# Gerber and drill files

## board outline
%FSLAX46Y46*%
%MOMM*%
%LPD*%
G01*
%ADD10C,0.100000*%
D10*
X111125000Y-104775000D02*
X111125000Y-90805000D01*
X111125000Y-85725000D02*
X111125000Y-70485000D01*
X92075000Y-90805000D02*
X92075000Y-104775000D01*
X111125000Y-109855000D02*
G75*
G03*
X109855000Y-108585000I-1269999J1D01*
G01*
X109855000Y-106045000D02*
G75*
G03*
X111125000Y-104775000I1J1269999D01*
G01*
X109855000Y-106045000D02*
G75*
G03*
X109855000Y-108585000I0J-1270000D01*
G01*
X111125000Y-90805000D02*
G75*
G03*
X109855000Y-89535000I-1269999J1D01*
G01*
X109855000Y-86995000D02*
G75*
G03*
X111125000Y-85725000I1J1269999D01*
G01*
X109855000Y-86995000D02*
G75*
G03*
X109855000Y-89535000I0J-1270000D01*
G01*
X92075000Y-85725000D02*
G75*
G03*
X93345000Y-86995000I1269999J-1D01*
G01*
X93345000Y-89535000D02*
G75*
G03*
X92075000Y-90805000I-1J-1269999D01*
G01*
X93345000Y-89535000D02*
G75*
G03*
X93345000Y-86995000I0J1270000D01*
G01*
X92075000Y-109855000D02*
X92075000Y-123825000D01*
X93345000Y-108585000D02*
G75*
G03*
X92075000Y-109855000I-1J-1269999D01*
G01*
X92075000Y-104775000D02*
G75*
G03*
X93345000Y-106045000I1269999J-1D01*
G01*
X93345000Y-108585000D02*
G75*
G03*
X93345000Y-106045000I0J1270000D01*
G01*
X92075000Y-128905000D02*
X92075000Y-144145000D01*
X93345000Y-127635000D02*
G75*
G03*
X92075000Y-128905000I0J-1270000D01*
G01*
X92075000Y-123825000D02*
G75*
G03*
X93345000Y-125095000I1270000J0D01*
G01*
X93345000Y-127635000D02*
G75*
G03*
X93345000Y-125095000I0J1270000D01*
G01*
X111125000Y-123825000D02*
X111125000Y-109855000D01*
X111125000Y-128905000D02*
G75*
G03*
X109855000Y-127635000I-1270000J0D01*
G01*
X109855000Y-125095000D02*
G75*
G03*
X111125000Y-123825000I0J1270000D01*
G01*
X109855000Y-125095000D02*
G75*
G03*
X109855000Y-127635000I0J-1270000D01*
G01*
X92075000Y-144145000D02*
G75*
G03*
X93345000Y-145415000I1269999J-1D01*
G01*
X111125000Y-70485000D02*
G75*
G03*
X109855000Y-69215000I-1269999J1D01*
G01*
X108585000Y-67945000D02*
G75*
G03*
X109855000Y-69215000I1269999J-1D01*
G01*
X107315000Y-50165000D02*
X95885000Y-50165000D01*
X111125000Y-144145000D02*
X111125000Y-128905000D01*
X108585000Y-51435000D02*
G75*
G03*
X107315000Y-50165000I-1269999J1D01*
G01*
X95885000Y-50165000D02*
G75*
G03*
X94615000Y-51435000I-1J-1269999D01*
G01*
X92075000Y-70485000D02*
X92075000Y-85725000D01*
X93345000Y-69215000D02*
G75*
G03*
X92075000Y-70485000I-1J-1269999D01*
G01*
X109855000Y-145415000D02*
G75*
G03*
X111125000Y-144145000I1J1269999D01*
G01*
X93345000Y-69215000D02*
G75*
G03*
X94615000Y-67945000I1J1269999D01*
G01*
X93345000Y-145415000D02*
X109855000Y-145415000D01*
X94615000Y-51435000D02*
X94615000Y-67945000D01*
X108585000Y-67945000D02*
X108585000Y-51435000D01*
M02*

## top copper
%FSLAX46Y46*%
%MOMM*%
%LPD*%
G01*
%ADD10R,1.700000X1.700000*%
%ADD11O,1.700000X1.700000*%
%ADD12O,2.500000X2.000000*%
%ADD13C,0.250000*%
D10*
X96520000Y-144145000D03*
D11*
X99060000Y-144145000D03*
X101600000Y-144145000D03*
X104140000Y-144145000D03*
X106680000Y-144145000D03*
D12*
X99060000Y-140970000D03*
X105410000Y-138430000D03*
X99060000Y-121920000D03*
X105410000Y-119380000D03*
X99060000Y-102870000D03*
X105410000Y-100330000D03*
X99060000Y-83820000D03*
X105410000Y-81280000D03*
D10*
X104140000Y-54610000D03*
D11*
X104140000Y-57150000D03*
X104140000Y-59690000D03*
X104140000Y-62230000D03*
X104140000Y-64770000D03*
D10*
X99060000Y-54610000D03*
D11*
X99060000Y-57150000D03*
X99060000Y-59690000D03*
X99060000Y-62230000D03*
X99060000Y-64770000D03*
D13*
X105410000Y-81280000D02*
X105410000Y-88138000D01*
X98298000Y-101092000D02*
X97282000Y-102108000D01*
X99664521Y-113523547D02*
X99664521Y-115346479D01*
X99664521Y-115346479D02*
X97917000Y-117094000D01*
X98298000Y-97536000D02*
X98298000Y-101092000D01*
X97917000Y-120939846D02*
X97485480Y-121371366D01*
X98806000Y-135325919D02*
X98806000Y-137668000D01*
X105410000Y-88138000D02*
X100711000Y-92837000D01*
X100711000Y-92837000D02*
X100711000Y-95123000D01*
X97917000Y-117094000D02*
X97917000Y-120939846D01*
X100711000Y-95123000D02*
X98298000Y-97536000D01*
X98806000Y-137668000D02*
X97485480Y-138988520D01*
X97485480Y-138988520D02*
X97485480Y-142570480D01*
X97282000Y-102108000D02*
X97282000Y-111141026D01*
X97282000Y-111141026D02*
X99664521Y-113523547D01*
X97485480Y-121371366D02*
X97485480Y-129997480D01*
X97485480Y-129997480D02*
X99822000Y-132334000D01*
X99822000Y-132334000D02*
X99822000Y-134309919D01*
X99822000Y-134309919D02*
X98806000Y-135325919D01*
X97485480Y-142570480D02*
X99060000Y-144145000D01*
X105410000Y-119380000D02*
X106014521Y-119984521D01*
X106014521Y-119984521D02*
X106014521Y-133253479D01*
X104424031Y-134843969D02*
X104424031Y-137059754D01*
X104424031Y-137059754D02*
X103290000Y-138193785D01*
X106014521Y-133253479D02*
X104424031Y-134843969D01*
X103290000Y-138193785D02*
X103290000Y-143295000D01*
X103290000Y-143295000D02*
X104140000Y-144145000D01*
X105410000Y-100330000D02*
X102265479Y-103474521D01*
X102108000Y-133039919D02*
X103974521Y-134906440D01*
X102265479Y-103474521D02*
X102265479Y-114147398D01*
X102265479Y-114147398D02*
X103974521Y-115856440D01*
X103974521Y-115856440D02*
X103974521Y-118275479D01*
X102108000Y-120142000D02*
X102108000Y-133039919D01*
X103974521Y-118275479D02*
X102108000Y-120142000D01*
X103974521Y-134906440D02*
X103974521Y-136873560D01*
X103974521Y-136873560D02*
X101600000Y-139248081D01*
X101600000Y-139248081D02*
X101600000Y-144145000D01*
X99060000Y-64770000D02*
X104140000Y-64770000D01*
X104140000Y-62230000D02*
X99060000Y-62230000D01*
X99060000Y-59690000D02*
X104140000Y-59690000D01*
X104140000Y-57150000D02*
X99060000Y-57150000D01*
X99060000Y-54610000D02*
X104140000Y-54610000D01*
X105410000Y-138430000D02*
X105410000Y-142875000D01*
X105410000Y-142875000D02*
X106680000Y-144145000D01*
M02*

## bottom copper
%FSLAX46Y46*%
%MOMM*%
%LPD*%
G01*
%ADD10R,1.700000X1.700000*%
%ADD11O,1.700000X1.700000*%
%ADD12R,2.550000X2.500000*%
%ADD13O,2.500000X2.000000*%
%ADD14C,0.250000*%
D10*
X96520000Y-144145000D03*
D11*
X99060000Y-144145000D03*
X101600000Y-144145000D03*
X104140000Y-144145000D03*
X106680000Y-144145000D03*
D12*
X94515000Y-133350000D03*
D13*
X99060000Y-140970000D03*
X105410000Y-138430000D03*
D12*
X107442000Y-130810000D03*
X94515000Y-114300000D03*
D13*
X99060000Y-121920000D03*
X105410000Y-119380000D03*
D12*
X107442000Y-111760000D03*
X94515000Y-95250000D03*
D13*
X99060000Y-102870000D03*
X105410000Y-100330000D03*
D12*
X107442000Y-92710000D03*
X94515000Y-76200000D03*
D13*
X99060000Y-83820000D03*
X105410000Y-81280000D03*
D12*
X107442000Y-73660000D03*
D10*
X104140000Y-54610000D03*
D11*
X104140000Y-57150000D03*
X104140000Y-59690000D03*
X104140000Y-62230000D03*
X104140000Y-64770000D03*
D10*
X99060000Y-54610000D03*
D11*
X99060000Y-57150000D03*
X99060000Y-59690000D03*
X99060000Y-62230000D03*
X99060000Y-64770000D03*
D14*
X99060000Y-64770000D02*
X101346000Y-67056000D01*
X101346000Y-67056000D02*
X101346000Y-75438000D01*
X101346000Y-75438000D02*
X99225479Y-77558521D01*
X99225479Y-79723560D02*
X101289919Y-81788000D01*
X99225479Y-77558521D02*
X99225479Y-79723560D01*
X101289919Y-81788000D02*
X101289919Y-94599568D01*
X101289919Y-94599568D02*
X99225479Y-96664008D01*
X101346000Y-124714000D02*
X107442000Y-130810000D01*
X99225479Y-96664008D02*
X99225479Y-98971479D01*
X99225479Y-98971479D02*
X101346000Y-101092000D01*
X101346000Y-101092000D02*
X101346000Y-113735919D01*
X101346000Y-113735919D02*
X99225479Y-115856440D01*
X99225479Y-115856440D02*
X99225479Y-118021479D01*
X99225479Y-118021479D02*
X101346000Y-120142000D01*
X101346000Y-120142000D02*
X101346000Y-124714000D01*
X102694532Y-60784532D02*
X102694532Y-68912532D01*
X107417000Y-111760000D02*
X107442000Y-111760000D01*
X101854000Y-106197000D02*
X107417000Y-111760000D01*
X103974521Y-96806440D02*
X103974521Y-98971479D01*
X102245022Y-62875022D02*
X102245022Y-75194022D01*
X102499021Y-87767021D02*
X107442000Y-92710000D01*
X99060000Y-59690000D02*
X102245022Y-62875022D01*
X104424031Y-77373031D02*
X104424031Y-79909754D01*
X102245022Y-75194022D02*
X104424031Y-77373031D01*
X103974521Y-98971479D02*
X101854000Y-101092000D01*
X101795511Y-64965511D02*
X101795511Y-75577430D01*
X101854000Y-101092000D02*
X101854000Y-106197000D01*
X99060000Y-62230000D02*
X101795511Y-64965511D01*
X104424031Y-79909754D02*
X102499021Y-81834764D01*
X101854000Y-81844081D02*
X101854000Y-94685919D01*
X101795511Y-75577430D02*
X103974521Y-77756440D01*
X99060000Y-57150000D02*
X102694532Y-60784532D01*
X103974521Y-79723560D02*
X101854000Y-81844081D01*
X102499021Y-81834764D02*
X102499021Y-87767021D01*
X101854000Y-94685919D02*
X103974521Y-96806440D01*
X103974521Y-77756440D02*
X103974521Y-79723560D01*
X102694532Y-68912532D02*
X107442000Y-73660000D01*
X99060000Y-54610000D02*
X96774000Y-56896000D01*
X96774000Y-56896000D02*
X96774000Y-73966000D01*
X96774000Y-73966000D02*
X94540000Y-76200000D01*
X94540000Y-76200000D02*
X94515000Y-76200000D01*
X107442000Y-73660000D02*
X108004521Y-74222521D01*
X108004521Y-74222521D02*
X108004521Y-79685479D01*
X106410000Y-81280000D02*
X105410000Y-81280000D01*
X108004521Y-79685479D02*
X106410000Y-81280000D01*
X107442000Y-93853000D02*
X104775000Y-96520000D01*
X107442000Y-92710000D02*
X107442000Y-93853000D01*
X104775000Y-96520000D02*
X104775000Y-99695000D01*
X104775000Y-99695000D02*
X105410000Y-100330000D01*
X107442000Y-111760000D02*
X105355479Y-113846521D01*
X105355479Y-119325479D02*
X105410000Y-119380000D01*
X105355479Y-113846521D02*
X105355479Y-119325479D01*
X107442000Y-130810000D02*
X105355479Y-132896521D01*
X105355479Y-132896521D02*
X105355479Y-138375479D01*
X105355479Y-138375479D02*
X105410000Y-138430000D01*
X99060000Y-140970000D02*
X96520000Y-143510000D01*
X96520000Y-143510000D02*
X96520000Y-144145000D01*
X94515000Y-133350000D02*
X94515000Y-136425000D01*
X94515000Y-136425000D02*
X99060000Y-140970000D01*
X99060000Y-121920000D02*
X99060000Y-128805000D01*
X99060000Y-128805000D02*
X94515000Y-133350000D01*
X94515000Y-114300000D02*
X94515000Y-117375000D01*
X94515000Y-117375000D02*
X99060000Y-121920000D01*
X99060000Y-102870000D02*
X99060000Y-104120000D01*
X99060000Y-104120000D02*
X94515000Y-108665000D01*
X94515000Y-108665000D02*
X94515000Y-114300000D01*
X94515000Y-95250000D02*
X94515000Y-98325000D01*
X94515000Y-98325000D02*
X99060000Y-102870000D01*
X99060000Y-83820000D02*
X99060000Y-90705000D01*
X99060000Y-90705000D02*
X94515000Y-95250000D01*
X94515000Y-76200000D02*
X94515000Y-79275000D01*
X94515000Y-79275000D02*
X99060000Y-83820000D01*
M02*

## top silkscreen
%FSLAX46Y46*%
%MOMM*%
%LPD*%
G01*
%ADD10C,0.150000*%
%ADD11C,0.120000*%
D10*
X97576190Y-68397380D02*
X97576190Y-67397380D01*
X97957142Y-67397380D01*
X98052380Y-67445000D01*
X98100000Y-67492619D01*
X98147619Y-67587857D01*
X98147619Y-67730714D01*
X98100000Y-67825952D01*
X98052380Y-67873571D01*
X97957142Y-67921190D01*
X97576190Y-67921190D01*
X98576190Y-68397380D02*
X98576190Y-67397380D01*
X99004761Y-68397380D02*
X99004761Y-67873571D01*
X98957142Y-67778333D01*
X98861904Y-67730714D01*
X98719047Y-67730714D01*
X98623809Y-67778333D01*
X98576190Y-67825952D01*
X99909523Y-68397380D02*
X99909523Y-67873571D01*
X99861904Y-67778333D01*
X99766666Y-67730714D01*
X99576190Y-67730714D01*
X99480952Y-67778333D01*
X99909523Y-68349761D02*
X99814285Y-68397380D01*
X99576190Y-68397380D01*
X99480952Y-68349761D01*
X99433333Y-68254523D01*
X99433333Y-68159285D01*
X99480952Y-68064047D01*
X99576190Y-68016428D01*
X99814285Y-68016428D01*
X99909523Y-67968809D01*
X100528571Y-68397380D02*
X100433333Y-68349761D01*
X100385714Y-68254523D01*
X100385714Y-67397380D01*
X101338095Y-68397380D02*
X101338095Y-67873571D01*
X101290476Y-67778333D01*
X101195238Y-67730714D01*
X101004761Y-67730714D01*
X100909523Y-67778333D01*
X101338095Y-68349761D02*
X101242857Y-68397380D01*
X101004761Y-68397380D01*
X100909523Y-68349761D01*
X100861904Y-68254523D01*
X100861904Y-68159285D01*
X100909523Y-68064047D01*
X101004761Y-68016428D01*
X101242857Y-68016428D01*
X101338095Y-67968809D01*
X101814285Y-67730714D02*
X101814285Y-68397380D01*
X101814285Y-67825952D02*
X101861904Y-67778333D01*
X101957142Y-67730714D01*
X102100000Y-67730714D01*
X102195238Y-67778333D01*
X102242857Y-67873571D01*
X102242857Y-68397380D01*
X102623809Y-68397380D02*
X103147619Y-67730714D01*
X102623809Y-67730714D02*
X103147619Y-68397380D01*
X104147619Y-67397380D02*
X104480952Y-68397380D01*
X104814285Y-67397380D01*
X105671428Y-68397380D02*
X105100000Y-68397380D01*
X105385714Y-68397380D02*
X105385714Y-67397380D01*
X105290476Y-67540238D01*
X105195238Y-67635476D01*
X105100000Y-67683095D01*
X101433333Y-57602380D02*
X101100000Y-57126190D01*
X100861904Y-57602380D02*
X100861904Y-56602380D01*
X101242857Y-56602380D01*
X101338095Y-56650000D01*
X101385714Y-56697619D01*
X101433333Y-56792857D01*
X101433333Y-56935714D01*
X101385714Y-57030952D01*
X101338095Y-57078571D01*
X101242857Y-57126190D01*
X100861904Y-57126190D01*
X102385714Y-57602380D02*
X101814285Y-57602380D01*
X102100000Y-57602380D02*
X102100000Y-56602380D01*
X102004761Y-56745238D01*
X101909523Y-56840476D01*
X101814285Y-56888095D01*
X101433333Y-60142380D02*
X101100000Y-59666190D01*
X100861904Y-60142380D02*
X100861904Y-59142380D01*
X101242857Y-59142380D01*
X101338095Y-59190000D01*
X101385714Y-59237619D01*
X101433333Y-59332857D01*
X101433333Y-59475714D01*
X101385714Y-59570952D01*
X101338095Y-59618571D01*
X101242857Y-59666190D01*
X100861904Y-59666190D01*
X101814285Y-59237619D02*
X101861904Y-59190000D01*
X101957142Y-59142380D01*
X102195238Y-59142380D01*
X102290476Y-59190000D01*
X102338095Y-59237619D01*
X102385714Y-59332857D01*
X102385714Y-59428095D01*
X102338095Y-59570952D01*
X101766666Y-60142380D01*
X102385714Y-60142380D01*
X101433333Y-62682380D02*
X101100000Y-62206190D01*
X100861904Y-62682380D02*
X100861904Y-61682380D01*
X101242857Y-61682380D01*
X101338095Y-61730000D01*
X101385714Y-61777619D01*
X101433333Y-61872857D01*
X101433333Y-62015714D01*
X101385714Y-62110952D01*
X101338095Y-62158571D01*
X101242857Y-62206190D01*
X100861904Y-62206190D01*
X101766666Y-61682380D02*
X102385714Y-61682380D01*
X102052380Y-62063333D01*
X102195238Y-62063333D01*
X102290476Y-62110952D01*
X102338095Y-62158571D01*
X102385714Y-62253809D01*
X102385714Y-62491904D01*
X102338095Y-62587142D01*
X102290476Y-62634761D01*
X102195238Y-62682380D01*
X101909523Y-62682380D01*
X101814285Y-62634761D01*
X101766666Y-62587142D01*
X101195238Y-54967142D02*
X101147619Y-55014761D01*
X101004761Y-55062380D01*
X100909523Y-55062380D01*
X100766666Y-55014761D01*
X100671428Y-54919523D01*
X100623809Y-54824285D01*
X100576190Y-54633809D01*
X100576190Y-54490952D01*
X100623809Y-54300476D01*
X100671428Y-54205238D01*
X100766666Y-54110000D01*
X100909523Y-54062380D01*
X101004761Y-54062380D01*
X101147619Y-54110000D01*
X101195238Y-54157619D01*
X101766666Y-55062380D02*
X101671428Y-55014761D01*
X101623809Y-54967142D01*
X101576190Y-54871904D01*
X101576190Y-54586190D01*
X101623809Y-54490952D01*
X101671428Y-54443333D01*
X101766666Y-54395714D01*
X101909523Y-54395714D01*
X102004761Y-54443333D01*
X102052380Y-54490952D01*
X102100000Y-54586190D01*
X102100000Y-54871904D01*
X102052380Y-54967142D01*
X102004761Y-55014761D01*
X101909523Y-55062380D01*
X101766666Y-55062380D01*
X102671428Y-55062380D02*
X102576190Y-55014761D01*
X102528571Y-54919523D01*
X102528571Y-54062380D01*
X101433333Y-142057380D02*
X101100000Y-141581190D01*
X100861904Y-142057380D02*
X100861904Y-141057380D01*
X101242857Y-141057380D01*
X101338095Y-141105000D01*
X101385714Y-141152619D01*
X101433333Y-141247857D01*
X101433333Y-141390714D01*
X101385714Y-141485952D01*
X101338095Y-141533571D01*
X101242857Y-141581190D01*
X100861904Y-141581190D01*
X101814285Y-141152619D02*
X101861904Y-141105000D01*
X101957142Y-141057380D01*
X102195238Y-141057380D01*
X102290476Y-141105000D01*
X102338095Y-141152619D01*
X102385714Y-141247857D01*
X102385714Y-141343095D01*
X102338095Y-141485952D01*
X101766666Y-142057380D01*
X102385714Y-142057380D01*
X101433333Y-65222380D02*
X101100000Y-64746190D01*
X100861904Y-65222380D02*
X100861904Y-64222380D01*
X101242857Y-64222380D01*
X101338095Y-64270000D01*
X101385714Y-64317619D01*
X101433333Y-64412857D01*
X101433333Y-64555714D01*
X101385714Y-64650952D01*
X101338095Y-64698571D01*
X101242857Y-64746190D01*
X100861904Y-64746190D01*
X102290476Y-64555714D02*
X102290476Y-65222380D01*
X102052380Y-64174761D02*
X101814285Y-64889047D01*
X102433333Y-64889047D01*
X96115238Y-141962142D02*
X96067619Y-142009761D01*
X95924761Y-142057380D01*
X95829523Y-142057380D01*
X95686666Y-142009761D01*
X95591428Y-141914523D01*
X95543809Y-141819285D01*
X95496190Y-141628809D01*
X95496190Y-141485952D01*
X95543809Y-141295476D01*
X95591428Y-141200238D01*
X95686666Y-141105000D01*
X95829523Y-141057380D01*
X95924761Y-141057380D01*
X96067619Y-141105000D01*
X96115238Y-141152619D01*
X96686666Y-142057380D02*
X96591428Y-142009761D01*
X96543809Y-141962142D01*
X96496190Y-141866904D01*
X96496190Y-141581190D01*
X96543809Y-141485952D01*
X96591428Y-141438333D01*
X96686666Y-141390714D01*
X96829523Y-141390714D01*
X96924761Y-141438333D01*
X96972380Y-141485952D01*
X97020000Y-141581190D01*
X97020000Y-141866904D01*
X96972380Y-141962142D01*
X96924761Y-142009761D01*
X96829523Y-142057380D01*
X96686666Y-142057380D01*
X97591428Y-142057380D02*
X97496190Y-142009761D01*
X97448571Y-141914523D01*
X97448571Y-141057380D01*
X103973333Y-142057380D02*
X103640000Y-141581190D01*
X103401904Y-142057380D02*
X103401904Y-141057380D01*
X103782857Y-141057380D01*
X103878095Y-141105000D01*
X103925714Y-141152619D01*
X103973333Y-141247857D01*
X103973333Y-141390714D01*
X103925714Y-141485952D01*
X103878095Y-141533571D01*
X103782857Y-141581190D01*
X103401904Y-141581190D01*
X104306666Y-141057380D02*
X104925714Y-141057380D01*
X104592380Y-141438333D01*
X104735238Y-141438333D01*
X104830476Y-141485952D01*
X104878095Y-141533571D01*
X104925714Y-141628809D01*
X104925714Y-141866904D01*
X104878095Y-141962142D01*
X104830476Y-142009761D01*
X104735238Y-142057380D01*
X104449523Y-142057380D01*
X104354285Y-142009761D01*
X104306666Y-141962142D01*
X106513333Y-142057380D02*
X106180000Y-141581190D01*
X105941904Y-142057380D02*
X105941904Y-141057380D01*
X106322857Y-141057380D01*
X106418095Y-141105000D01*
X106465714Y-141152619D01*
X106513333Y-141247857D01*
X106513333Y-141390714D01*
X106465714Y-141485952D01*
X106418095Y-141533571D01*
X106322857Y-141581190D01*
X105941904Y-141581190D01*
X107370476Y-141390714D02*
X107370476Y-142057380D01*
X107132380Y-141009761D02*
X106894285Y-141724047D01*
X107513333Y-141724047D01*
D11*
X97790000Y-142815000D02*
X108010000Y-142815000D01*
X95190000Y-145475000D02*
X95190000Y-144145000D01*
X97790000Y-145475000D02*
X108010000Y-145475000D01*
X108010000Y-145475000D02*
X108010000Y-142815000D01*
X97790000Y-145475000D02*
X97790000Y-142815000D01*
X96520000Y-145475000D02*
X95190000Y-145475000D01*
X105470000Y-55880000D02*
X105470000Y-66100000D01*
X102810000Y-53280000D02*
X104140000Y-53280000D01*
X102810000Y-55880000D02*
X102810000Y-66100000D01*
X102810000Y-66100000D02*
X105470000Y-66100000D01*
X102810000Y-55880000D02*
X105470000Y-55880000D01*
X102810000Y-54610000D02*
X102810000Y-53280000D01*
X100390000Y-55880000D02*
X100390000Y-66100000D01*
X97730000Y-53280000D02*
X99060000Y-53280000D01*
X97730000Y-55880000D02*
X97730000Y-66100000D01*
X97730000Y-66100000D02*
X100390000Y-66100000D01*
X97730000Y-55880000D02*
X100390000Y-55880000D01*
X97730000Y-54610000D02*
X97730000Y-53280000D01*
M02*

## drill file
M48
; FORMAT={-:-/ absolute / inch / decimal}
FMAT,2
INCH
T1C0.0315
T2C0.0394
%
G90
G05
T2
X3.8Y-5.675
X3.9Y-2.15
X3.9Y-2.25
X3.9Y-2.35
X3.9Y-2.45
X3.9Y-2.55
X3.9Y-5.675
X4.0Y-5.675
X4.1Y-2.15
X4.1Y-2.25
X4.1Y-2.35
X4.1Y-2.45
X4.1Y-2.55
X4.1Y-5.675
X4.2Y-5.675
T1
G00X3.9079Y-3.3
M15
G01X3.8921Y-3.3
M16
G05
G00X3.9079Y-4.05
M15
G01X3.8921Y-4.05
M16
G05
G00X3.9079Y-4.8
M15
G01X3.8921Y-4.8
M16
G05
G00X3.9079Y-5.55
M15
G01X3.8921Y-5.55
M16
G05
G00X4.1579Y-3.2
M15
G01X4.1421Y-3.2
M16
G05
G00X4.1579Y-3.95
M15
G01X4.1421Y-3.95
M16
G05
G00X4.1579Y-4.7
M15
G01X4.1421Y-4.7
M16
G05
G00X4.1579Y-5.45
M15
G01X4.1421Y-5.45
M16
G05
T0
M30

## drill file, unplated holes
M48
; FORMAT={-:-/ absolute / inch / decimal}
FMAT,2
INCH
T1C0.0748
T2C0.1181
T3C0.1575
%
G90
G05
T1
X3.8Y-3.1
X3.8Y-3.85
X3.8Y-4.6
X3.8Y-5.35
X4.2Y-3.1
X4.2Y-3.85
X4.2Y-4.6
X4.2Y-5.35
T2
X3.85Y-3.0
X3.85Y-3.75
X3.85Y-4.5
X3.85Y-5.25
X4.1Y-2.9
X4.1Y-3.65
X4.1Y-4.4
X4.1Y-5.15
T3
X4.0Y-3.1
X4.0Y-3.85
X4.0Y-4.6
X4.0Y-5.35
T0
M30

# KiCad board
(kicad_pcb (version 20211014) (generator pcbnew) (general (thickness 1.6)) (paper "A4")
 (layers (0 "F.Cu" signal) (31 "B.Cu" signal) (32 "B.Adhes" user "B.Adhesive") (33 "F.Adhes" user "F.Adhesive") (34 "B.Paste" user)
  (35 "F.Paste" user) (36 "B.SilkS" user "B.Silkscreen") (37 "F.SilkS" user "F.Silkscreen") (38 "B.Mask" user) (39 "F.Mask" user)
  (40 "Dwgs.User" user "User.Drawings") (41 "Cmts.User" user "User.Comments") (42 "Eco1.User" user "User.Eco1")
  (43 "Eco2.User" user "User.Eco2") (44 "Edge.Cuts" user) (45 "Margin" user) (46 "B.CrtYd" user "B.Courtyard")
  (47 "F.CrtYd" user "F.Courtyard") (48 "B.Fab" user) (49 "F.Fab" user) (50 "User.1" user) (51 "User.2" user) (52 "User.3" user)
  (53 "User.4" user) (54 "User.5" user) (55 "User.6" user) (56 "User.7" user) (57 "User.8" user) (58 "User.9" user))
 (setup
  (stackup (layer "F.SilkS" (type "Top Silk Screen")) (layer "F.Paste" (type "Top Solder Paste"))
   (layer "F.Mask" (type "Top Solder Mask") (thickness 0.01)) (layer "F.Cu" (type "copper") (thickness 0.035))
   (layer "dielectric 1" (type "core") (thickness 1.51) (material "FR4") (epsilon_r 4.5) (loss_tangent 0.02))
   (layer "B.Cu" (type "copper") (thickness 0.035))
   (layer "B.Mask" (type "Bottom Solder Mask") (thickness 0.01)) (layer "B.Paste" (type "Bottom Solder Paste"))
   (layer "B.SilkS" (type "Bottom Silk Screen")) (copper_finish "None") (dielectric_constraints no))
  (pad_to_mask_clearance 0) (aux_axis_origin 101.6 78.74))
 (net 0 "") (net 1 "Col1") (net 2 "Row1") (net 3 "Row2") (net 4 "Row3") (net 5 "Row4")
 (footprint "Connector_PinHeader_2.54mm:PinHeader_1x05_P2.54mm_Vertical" (layer "F.Cu") (at 104.14 54.61)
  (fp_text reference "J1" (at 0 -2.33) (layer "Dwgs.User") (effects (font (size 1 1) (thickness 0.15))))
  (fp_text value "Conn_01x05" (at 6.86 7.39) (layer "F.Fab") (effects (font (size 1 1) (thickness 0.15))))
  (fp_line (start -1.33 -1.33) (end 0 -1.33) (layer "F.SilkS") (width 0.12))
  (fp_line (start -1.33 1.27) (end -1.33 11.49) (layer "F.SilkS") (width 0.12))
  (fp_line (start -1.33 11.49) (end 1.33 11.49) (layer "F.SilkS") (width 0.12))
  (fp_line (start -1.33 0) (end -1.33 -1.33) (layer "F.SilkS") (width 0.12))
  (fp_line (start -1.33 1.27) (end 1.33 1.27) (layer "F.SilkS") (width 0.12))
  (fp_line (start 1.33 1.27) (end 1.33 11.49) (layer "F.SilkS") (width 0.12))
  (pad "1" thru_hole rect (at 0 0) (size 1.7 1.7) (drill 1) (layers *.Cu *.Mask) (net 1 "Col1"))
  (pad "2" thru_hole oval (at 0 2.54) (size 1.7 1.7) (drill 1) (layers *.Cu *.Mask) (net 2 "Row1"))
  (pad "3" thru_hole oval (at 0 5.08) (size 1.7 1.7) (drill 1) (layers *.Cu *.Mask) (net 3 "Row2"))
  (pad "4" thru_hole oval (at 0 7.62) (size 1.7 1.7) (drill 1) (layers *.Cu *.Mask) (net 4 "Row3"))
  (pad "5" thru_hole oval (at 0 10.16) (size 1.7 1.7) (drill 1) (layers *.Cu *.Mask) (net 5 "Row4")))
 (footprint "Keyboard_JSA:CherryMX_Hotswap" (layer "F.Cu") (at 101.6 116.84)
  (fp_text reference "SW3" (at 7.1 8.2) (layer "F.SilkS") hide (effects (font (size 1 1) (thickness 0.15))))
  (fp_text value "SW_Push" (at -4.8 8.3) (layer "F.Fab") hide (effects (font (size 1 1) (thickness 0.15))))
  (pad "" np_thru_hole circle (at -5.08 0) (size 1.9 1.9) (drill 1.9) (layers *.Cu *.Mask))
  (pad "" np_thru_hole circle (at 2.54 -5.08) (size 3 3) (drill 3) (layers *.Cu *.Mask))
  (pad "" np_thru_hole circle (at 0 0) (size 4 4) (drill 4) (layers F&B.Cu *.Mask))
  (pad "" np_thru_hole circle (at 5.08 0) (size 1.9 1.9) (drill 1.9) (layers *.Cu *.Mask))
  (pad "" np_thru_hole circle (at -3.81 -2.54) (size 3 3) (drill 3) (layers *.Cu *.Mask))
  (pad "1" thru_hole oval (at -2.54 5.08 180) (size 2.5 2) (drill oval 1.2 0.8) (layers *.Cu *.Mask) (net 1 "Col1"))
  (pad "1" smd rect (at -7.085 -2.54 180) (size 2.55 2.5) (layers "B.Cu" "B.Paste" "B.Mask") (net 1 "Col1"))
  (pad "2" thru_hole oval (at 3.81 2.54 180) (size 2.5 2) (drill oval 1.2 0.8) (layers *.Cu *.Mask) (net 4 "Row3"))
  (pad "2" smd rect (at 5.842 -5.08 180) (size 2.55 2.5) (layers "B.Cu" "B.Paste" "B.Mask") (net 4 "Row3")))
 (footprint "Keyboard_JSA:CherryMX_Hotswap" (layer "F.Cu") (at 101.6 135.89)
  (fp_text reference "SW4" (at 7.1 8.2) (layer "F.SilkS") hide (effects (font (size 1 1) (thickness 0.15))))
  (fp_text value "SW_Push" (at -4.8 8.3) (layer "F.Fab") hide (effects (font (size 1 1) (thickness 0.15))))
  (pad "" np_thru_hole circle (at 0 0) (size 4 4) (drill 4) (layers F&B.Cu *.Mask))
  (pad "" np_thru_hole circle (at -3.81 -2.54) (size 3 3) (drill 3) (layers *.Cu *.Mask))
  (pad "" np_thru_hole circle (at -5.08 0) (size 1.9 1.9) (drill 1.9) (layers *.Cu *.Mask))
  (pad "" np_thru_hole circle (at 2.54 -5.08) (size 3 3) (drill 3) (layers *.Cu *.Mask))
  (pad "" np_thru_hole circle (at 5.08 0) (size 1.9 1.9) (drill 1.9) (layers *.Cu *.Mask))
  (pad "1" smd rect (at -7.085 -2.54 180) (size 2.55 2.5) (layers "B.Cu" "B.Paste" "B.Mask") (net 1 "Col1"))
  (pad "1" thru_hole oval (at -2.54 5.08 180) (size 2.5 2) (drill oval 1.2 0.8) (layers *.Cu *.Mask) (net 1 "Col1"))
  (pad "2" smd rect (at 5.842 -5.08 180) (size 2.55 2.5) (layers "B.Cu" "B.Paste" "B.Mask") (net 5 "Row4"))
  (pad "2" thru_hole oval (at 3.81 2.54 180) (size 2.5 2) (drill oval 1.2 0.8) (layers *.Cu *.Mask) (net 5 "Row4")))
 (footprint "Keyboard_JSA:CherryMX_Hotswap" (layer "F.Cu") (at 101.6 97.79)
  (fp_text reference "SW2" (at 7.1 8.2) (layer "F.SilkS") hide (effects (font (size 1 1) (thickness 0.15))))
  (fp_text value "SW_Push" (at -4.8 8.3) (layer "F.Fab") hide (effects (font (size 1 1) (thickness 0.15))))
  (pad "" np_thru_hole circle (at -5.08 0) (size 1.9 1.9) (drill 1.9) (layers *.Cu *.Mask))
  (pad "" np_thru_hole circle (at 5.08 0) (size 1.9 1.9) (drill 1.9) (layers *.Cu *.Mask))
  (pad "" np_thru_hole circle (at 0 0) (size 4 4) (drill 4) (layers F&B.Cu *.Mask))
  (pad "" np_thru_hole circle (at -3.81 -2.54) (size 3 3) (drill 3) (layers *.Cu *.Mask))
  (pad "" np_thru_hole circle (at 2.54 -5.08) (size 3 3) (drill 3) (layers *.Cu *.Mask))
  (pad "1" smd rect (at -7.085 -2.54 180) (size 2.55 2.5) (layers "B.Cu" "B.Paste" "B.Mask") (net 1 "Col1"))
  (pad "1" thru_hole oval (at -2.54 5.08 180) (size 2.5 2) (drill oval 1.2 0.8) (layers *.Cu *.Mask) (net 1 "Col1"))
  (pad "2" thru_hole oval (at 3.81 2.54 180) (size 2.5 2) (drill oval 1.2 0.8) (layers *.Cu *.Mask) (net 3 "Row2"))
  (pad "2" smd rect (at 5.842 -5.08 180) (size 2.55 2.5) (layers "B.Cu" "B.Paste" "B.Mask") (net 3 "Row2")))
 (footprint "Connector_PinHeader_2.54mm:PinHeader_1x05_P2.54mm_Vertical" (layer "F.Cu") (at 99.06 54.61)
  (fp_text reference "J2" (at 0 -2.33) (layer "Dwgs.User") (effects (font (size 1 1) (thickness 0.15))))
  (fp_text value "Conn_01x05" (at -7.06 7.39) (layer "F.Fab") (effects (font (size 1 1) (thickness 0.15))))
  (fp_line (start -1.33 1.27) (end 1.33 1.27) (layer "F.SilkS") (width 0.12))
  (fp_line (start -1.33 11.49) (end 1.33 11.49) (layer "F.SilkS") (width 0.12))
  (fp_line (start 1.33 1.27) (end 1.33 11.49) (layer "F.SilkS") (width 0.12))
  (fp_line (start -1.33 -1.33) (end 0 -1.33) (layer "F.SilkS") (width 0.12))
  (fp_line (start -1.33 1.27) (end -1.33 11.49) (layer "F.SilkS") (width 0.12))
  (fp_line (start -1.33 0) (end -1.33 -1.33) (layer "F.SilkS") (width 0.12))
  (pad "1" thru_hole rect (at 0 0) (size 1.7 1.7) (drill 1) (layers *.Cu *.Mask) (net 1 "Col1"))
  (pad "2" thru_hole oval (at 0 2.54) (size 1.7 1.7) (drill 1) (layers *.Cu *.Mask) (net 2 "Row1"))
  (pad "3" thru_hole oval (at 0 5.08) (size 1.7 1.7) (drill 1) (layers *.Cu *.Mask) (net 3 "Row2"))
  (pad "4" thru_hole oval (at 0 7.62) (size 1.7 1.7) (drill 1) (layers *.Cu *.Mask) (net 4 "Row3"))
  (pad "5" thru_hole oval (at 0 10.16) (size 1.7 1.7) (drill 1) (layers *.Cu *.Mask) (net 5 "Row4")))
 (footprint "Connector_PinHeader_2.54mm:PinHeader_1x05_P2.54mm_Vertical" (layer "F.Cu") (at 96.52 144.145 90)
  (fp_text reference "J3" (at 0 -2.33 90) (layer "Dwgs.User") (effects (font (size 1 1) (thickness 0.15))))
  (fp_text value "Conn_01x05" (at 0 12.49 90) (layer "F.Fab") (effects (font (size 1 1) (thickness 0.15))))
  (fp_line (start -1.33 1.27) (end -1.33 11.49) (layer "F.SilkS") (width 0.12))
  (fp_line (start -1.33 0) (end -1.33 -1.33) (layer "F.SilkS") (width 0.12))
  (fp_line (start -1.33 -1.33) (end 0 -1.33) (layer "F.SilkS") (width 0.12))
  (fp_line (start -1.33 1.27) (end 1.33 1.27) (layer "F.SilkS") (width 0.12))
  (fp_line (start -1.33 11.49) (end 1.33 11.49) (layer "F.SilkS") (width 0.12))
  (fp_line (start 1.33 1.27) (end 1.33 11.49) (layer "F.SilkS") (width 0.12))
  (pad "1" thru_hole rect (at 0 0 90) (size 1.7 1.7) (drill 1) (layers *.Cu *.Mask) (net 1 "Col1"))
  (pad "2" thru_hole oval (at 0 2.54 90) (size 1.7 1.7) (drill 1) (layers *.Cu *.Mask) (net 2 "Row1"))
  (pad "3" thru_hole oval (at 0 5.08 90) (size 1.7 1.7) (drill 1) (layers *.Cu *.Mask) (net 3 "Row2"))
  (pad "4" thru_hole oval (at 0 7.62 90) (size 1.7 1.7) (drill 1) (layers *.Cu *.Mask) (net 4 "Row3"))
  (pad "5" thru_hole oval (at 0 10.16 90) (size 1.7 1.7) (drill 1) (layers *.Cu *.Mask) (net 5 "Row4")))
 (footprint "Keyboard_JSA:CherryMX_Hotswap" (layer "F.Cu") (at 101.6 78.74)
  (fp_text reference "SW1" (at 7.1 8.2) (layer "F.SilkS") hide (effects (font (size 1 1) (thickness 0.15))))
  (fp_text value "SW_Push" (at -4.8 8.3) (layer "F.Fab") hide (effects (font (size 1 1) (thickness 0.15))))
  (pad "" np_thru_hole circle (at -5.08 0) (size 1.9 1.9) (drill 1.9) (layers *.Cu *.Mask))
  (pad "" np_thru_hole circle (at 0 0) (size 4 4) (drill 4) (layers F&B.Cu *.Mask))
  (pad "" np_thru_hole circle (at -3.81 -2.54) (size 3 3) (drill 3) (layers *.Cu *.Mask))
  (pad "" np_thru_hole circle (at 5.08 0) (size 1.9 1.9) (drill 1.9) (layers *.Cu *.Mask))
  (pad "" np_thru_hole circle (at 2.54 -5.08) (size 3 3) (drill 3) (layers *.Cu *.Mask))
  (pad "1" thru_hole oval (at -2.54 5.08 180) (size 2.5 2) (drill oval 1.2 0.8) (layers *.Cu *.Mask) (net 1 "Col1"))
  (pad "1" smd rect (at -7.085 -2.54 180) (size 2.55 2.5) (layers "B.Cu" "B.Paste" "B.Mask") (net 1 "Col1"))
  (pad "2" smd rect (at 5.842 -5.08 180) (size 2.55 2.5) (layers "B.Cu" "B.Paste" "B.Mask") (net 2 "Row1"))
  (pad "2" thru_hole oval (at 3.81 2.54 180) (size 2.5 2) (drill oval 1.2 0.8) (layers *.Cu *.Mask) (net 2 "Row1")))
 (gr_arc (start 109.855 108.585) (mid 110.753026 108.956974) (end 111.125 109.855) (layer "Edge.Cuts") (width 0.1))
 (gr_arc (start 93.345 125.095) (mid 94.615 126.365) (end 93.345 127.635) (layer "Edge.Cuts") (width 0.1))
 (gr_arc (start 93.345 145.415) (mid 92.446974 145.043026) (end 92.075 144.145) (layer "Edge.Cuts") (width 0.1))
 (gr_arc (start 109.855 108.585) (mid 108.585 107.315) (end 109.855 106.045) (layer "Edge.Cuts") (width 0.1))
 (gr_arc (start 109.855 69.215) (mid 110.753026 69.586974) (end 111.125 70.485) (layer "Edge.Cuts") (width 0.1))
 (gr_arc (start 92.075 109.855) (mid 92.446974 108.956974) (end 93.345 108.585) (layer "Edge.Cuts") (width 0.1))
 (gr_arc (start 92.075 90.805) (mid 92.446974 89.906974) (end 93.345 89.535) (layer "Edge.Cuts") (width 0.1))
 (gr_arc (start 109.855 69.215) (mid 108.956974 68.843026) (end 108.585 67.945) (layer "Edge.Cuts") (width 0.1))
 (gr_line (start 107.315 50.165) (end 95.885 50.165) (layer "Edge.Cuts") (width 0.1))
 (gr_arc (start 93.345 86.995) (mid 92.446974 86.623026) (end 92.075 85.725) (layer "Edge.Cuts") (width 0.1))
 (gr_arc (start 111.125 85.725) (mid 110.753026 86.623026) (end 109.855 86.995) (layer "Edge.Cuts") (width 0.1))
 (gr_arc (start 93.345 125.095) (mid 92.446974 124.723026) (end 92.075 123.825) (layer "Edge.Cuts") (width 0.1))
 (gr_arc (start 111.125 104.775) (mid 110.753026 105.673026) (end 109.855 106.045) (layer "Edge.Cuts") (width 0.1))
 (gr_line (start 111.125 123.825) (end 111.125 109.855) (layer "Edge.Cuts") (width 0.1))
 (gr_line (start 111.125 85.725) (end 111.125 70.485) (layer "Edge.Cuts") (width 0.1))
 (gr_line (start 111.125 104.775) (end 111.125 90.805) (layer "Edge.Cuts") (width 0.1))
 (gr_line (start 111.125 144.145) (end 111.125 128.905) (layer "Edge.Cuts") (width 0.1))
 (gr_arc (start 109.855 127.635) (mid 108.585 126.365) (end 109.855 125.095) (layer "Edge.Cuts") (width 0.1))
 (gr_arc (start 93.345 106.045) (mid 94.615 107.315) (end 93.345 108.585) (layer "Edge.Cuts") (width 0.1))
 (gr_arc (start 109.855 89.535) (mid 110.753026 89.906974) (end 111.125 90.805) (layer "Edge.Cuts") (width 0.1))
 (gr_arc (start 107.315 50.165) (mid 108.213026 50.536974) (end 108.585 51.435) (layer "Edge.Cuts") (width 0.1))
 (gr_arc (start 94.615 51.435) (mid 94.986974 50.536974) (end 95.885 50.165) (layer "Edge.Cuts") (width 0.1))
 (gr_line (start 92.075 90.805) (end 92.075 104.775) (layer "Edge.Cuts") (width 0.1))
 (gr_line (start 92.075 109.855) (end 92.075 123.825) (layer "Edge.Cuts") (width 0.1))
 (gr_line (start 92.075 128.905) (end 92.075 144.145) (layer "Edge.Cuts") (width 0.1))
 (gr_line (start 92.075 70.485) (end 92.075 85.725) (layer "Edge.Cuts") (width 0.1))
 (gr_arc (start 92.075 70.485) (mid 92.446974 69.586974) (end 93.345 69.215) (layer "Edge.Cuts") (width 0.1))
 (gr_arc (start 92.075 128.905) (mid 92.446974 128.006974) (end 93.345 127.635) (layer "Edge.Cuts") (width 0.1))
 (gr_arc (start 111.125 144.145) (mid 110.753026 145.043026) (end 109.855 145.415) (layer "Edge.Cuts") (width 0.1))
 (gr_arc (start 94.615 67.945) (mid 94.243026 68.843026) (end 93.345 69.215) (layer "Edge.Cuts") (width 0.1))
 (gr_arc (start 109.855 127.635) (mid 110.753026 128.006974) (end 111.125 128.905) (layer "Edge.Cuts") (width 0.1))
 (gr_line (start 93.345 145.415) (end 109.855 145.415) (layer "Edge.Cuts") (width 0.1))
 (gr_arc (start 93.345 106.045) (mid 92.446974 105.673026) (end 92.075 104.775) (layer "Edge.Cuts") (width 0.1))
 (gr_arc (start 111.125 123.825) (mid 110.753026 124.723026) (end 109.855 125.095) (layer "Edge.Cuts") (width 0.1))
 (gr_arc (start 109.855 89.535) (mid 108.585 88.265) (end 109.855 86.995) (layer "Edge.Cuts") (width 0.1))
 (gr_line (start 94.615 51.435) (end 94.615 67.945) (layer "Edge.Cuts") (width 0.1))
 (gr_arc (start 93.345 86.995) (mid 94.615 88.265) (end 93.345 89.535) (layer "Edge.Cuts") (width 0.1))
 (gr_line (start 108.585 67.945) (end 108.585 51.435) (layer "Edge.Cuts") (width 0.1))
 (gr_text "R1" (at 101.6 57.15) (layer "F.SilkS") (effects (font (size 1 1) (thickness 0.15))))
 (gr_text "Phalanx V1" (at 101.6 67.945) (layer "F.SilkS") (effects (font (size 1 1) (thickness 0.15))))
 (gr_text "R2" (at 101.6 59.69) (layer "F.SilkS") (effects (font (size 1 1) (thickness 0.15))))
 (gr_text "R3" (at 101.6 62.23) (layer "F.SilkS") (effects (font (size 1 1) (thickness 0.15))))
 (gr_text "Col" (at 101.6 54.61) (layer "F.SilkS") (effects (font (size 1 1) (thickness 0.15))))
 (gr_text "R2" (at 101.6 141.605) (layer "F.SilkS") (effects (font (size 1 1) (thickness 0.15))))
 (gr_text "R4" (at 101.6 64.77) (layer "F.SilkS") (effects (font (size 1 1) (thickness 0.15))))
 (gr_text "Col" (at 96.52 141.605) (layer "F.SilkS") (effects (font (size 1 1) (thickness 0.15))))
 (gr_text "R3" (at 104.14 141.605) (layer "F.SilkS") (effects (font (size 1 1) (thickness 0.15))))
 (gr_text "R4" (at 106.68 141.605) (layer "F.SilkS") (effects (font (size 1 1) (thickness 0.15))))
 (segment (start 98.298 97.536) (end 98.298 101.092) (width 0.25) (layer "F.Cu") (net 2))
 (segment (start 97.48548 138.98852) (end 97.48548 142.57048) (width 0.25) (layer "F.Cu") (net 2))
 (segment (start 99.822 134.309919) (end 98.806 135.325919) (width 0.25) (layer "F.Cu") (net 2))
 (segment (start 105.41 88.138) (end 100.711 92.837) (width 0.25) (layer "F.Cu") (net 2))
 (segment (start 100.711 92.837) (end 100.711 95.123) (width 0.25) (layer "F.Cu") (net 2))
 (segment (start 99.664521 115.346479) (end 97.917 117.094) (width 0.25) (layer "F.Cu") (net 2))
 (segment (start 99.664521 113.523547) (end 99.664521 115.346479) (width 0.25) (layer "F.Cu") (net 2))
 (segment (start 97.917 117.094) (end 97.917 120.939846) (width 0.25) (layer "F.Cu") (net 2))
 (segment (start 100.711 95.123) (end 98.298 97.536) (width 0.25) (layer "F.Cu") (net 2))
 (segment (start 98.806 135.325919) (end 98.806 137.668) (width 0.25) (layer "F.Cu") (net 2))
 (segment (start 97.282 111.141026) (end 99.664521 113.523547) (width 0.25) (layer "F.Cu") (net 2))
 (segment (start 97.48548 129.99748) (end 99.822 132.334) (width 0.25) (layer "F.Cu") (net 2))
 (segment (start 98.806 137.668) (end 97.48548 138.98852) (width 0.25) (layer "F.Cu") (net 2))
 (segment (start 98.298 101.092) (end 97.282 102.108) (width 0.25) (layer "F.Cu") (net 2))
 (segment (start 105.41 81.28) (end 105.41 88.138) (width 0.25) (layer "F.Cu") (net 2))
 (segment (start 97.48548 142.57048) (end 99.06 144.145) (width 0.25) (layer "F.Cu") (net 2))
 (segment (start 104.14 57.15) (end 99.06 57.15) (width 0.25) (layer "F.Cu") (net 2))
 (segment (start 99.822 132.334) (end 99.822 134.309919) (width 0.25) (layer "F.Cu") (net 2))
 (segment (start 97.48548 121.371366) (end 97.48548 129.99748) (width 0.25) (layer "F.Cu") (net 2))
 (segment (start 97.917 120.939846) (end 97.48548 121.371366) (width 0.25) (layer "F.Cu") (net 2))
 (segment (start 97.282 102.108) (end 97.282 111.141026) (width 0.25) (layer "F.Cu") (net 2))
 (segment (start 107.442 73.66) (end 108.004521 74.222521) (width 0.25) (layer "B.Cu") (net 2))
 (segment (start 106.41 81.28) (end 105.41 81.28) (width 0.25) (layer "B.Cu") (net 2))
 (segment (start 108.004521 74.222521) (end 108.004521 79.685479) (width 0.25) (layer "B.Cu") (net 2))
 (segment (start 108.004521 79.685479) (end 106.41 81.28) (width 0.25) (layer "B.Cu") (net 2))
 (segment (start 102.694532 60.784532) (end 102.694532 68.912532) (width 0.25) (layer "B.Cu") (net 2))
 (segment (start 99.06 57.15) (end 102.694532 60.784532) (width 0.25) (layer "B.Cu") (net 2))
 (segment (start 102.694532 68.912532) (end 107.442 73.66) (width 0.25) (layer "B.Cu") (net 2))
 (segment (start 99.06 54.61) (end 104.14 54.61) (width 0.25) (layer "F.Cu") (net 1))
 (segment (start 99.06 104.12) (end 94.515 108.665) (width 0.25) (layer "B.Cu") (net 1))
 (segment (start 99.06 140.97) (end 96.52 143.51) (width 0.25) (layer "B.Cu") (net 1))
 (segment (start 96.774 56.896) (end 96.774 73.966) (width 0.25) (layer "B.Cu") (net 1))
 (segment (start 94.515 114.3) (end 94.515 117.375) (width 0.25) (layer "B.Cu") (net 1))
 (segment (start 94.515 76.2) (end 94.515 79.275) (width 0.25) (layer "B.Cu") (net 1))
 (segment (start 94.515 79.275) (end 99.06 83.82) (width 0.25) (layer "B.Cu") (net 1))
 (segment (start 94.515 136.425) (end 99.06 140.97) (width 0.25) (layer "B.Cu") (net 1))
 (segment (start 96.52 143.51) (end 96.52 144.145) (width 0.25) (layer "B.Cu") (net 1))
 (segment (start 99.06 90.705) (end 94.515 95.25) (width 0.25) (layer "B.Cu") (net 1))
 (segment (start 99.06 121.92) (end 99.06 128.805) (width 0.25) (layer "B.Cu") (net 1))
 (segment (start 94.515 133.35) (end 94.515 136.425) (width 0.25) (layer "B.Cu") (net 1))
 (segment (start 94.515 95.25) (end 94.515 98.325) (width 0.25) (layer "B.Cu") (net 1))
 (segment (start 96.774 73.966) (end 94.54 76.2) (width 0.25) (layer "B.Cu") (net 1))
 (segment (start 94.515 117.375) (end 99.06 121.92) (width 0.25) (layer "B.Cu") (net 1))
 (segment (start 99.06 128.805) (end 94.515 133.35) (width 0.25) (layer "B.Cu") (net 1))
 (segment (start 99.06 83.82) (end 99.06 90.705) (width 0.25) (layer "B.Cu") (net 1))
 (segment (start 94.54 76.2) (end 94.515 76.2) (width 0.25) (layer "B.Cu") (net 1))
 (segment (start 99.06 102.87) (end 99.06 104.12) (width 0.25) (layer "B.Cu") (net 1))
 (segment (start 94.515 98.325) (end 99.06 102.87) (width 0.25) (layer "B.Cu") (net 1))
 (segment (start 99.06 54.61) (end 96.774 56.896) (width 0.25) (layer "B.Cu") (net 1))
 (segment (start 94.515 108.665) (end 94.515 114.3) (width 0.25) (layer "B.Cu") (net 1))
 (segment (start 103.974521 118.275479) (end 102.108 120.142) (width 0.25) (layer "F.Cu") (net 3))
 (segment (start 103.974521 134.90644) (end 103.974521 136.87356) (width 0.25) (layer "F.Cu") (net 3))
 (segment (start 103.974521 136.87356) (end 101.6 139.248081) (width 0.25) (layer "F.Cu") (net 3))
 (segment (start 101.6 139.248081) (end 101.6 144.145) (width 0.25) (layer "F.Cu") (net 3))
 (segment (start 99.06 59.69) (end 104.14 59.69) (width 0.25) (layer "F.Cu") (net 3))
 (segment (start 102.265479 114.147398) (end 103.974521 115.85644) (width 0.25) (layer "F.Cu") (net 3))
 (segment (start 103.974521 115.85644) (end 103.974521 118.275479) (width 0.25) (layer "F.Cu") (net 3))
 (segment (start 105.41 100.33) (end 102.265479 103.474521) (width 0.25) (layer "F.Cu") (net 3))
 (segment (start 102.108 133.039919) (end 103.974521 134.90644) (width 0.25) (layer "F.Cu") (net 3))
 (segment (start 102.108 120.142) (end 102.108 133.039919) (width 0.25) (layer "F.Cu") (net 3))
 (segment (start 102.265479 103.474521) (end 102.265479 114.147398) (width 0.25) (layer "F.Cu") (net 3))
 (segment (start 102.245022 62.875022) (end 102.245022 75.194022) (width 0.25) (layer "B.Cu") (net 3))
 (segment (start 107.442 93.853) (end 104.775 96.52) (width 0.25) (layer "B.Cu") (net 3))
 (segment (start 99.06 59.69) (end 102.245022 62.875022) (width 0.25) (layer "B.Cu") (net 3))
 (segment (start 104.424031 77.373031) (end 104.424031 79.909754) (width 0.25) (layer "B.Cu") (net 3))
 (segment (start 102.499021 81.834764) (end 102.499021 87.767021) (width 0.25) (layer "B.Cu") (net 3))
 (segment (start 102.245022 75.194022) (end 104.424031 77.373031) (width 0.25) (layer "B.Cu") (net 3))
 (segment (start 104.775 99.695) (end 105.41 100.33) (width 0.25) (layer "B.Cu") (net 3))
 (segment (start 104.424031 79.909754) (end 102.499021 81.834764) (width 0.25) (layer "B.Cu") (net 3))
 (segment (start 102.499021 87.767021) (end 107.442 92.71) (width 0.25) (layer "B.Cu") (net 3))
 (segment (start 107.442 92.71) (end 107.442 93.853) (width 0.25) (layer "B.Cu") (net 3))
 (segment (start 104.775 96.52) (end 104.775 99.695) (width 0.25) (layer "B.Cu") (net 3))
 (segment (start 106.014521 119.984521) (end 106.014521 133.253479) (width 0.25) (layer "F.Cu") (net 4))
 (segment (start 105.41 119.38) (end 106.014521 119.984521) (width 0.25) (layer "F.Cu") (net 4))
 (segment (start 104.424031 134.843969) (end 104.424031 137.059754) (width 0.25) (layer "F.Cu") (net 4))
 (segment (start 103.29 138.193785) (end 103.29 143.295) (width 0.25) (layer "F.Cu") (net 4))
 (segment (start 106.014521 133.253479) (end 104.424031 134.843969) (width 0.25) (layer "F.Cu") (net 4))
 (segment (start 103.29 143.295) (end 104.14 144.145) (width 0.25) (layer "F.Cu") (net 4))
 (segment (start 104.424031 137.059754) (end 103.29 138.193785) (width 0.25) (layer "F.Cu") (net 4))
 (segment (start 104.14 62.23) (end 99.06 62.23) (width 0.25) (layer "F.Cu") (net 4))
 (segment (start 107.442 111.76) (end 105.355479 113.846521) (width 0.25) (layer "B.Cu") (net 4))
 (segment (start 101.795511 64.965511) (end 101.795511 75.57743) (width 0.25) (layer "B.Cu") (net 4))
 (segment (start 105.355479 113.846521) (end 105.355479 119.325479) (width 0.25) (layer "B.Cu") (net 4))
 (segment (start 101.854 81.844081) (end 101.854 94.685919) (width 0.25) (layer "B.Cu") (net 4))
 (segment (start 101.795511 75.57743) (end 103.974521 77.75644) (width 0.25) (layer "B.Cu") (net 4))
 (segment (start 103.974521 96.80644) (end 103.974521 98.971479) (width 0.25) (layer "B.Cu") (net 4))
 (segment (start 103.974521 77.75644) (end 103.974521 79.72356) (width 0.25) (layer "B.Cu") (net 4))
 (segment (start 103.974521 79.72356) (end 101.854 81.844081) (width 0.25) (layer "B.Cu") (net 4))
 (segment (start 103.974521 98.971479) (end 101.854 101.092) (width 0.25) (layer "B.Cu") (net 4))
 (segment (start 107.417 111.76) (end 107.442 111.76) (width 0.25) (layer "B.Cu") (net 4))
 (segment (start 101.854 94.685919) (end 103.974521 96.80644) (width 0.25) (layer "B.Cu") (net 4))
 (segment (start 101.854 101.092) (end 101.854 106.197) (width 0.25) (layer "B.Cu") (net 4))
 (segment (start 105.355479 119.325479) (end 105.41 119.38) (width 0.25) (layer "B.Cu") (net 4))
 (segment (start 99.06 62.23) (end 101.795511 64.965511) (width 0.25) (layer "B.Cu") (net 4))
 (segment (start 101.854 106.197) (end 107.417 111.76) (width 0.25) (layer "B.Cu") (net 4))
 (segment (start 105.41 142.875) (end 106.68 144.145) (width 0.25) (layer "F.Cu") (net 5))
 (segment (start 99.06 64.77) (end 104.14 64.77) (width 0.25) (layer "F.Cu") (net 5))
 (segment (start 105.41 138.43) (end 105.41 142.875) (width 0.25) (layer "F.Cu") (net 5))
 (segment (start 101.346 124.714) (end 107.442 130.81) (width 0.25) (layer "B.Cu") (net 5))
 (segment (start 99.225479 77.558521) (end 99.225479 79.72356) (width 0.25) (layer "B.Cu") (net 5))
 (segment (start 101.346 101.092) (end 101.346 113.735919) (width 0.25) (layer "B.Cu") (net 5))
 (segment (start 101.346 67.056) (end 101.346 75.438) (width 0.25) (layer "B.Cu") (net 5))
 (segment (start 101.289919 94.599568) (end 99.225479 96.664008) (width 0.25) (layer "B.Cu") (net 5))
 (segment (start 99.225479 98.971479) (end 101.346 101.092) (width 0.25) (layer "B.Cu") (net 5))
 (segment (start 99.225479 96.664008) (end 99.225479 98.971479) (width 0.25) (layer "B.Cu") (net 5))
 (segment (start 101.289919 81.788) (end 101.289919 94.599568) (width 0.25) (layer "B.Cu") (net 5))
 (segment (start 105.355479 132.896521) (end 105.355479 138.375479) (width 0.25) (layer "B.Cu") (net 5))
 (segment (start 99.225479 79.72356) (end 101.289919 81.788) (width 0.25) (layer "B.Cu") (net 5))
 (segment (start 99.225479 115.85644) (end 99.225479 118.021479) (width 0.25) (layer "B.Cu") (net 5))
 (segment (start 107.442 130.81) (end 105.355479 132.896521) (width 0.25) (layer "B.Cu") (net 5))
 (segment (start 99.225479 118.021479) (end 101.346 120.142) (width 0.25) (layer "B.Cu") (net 5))
 (segment (start 101.346 75.438) (end 99.225479 77.558521) (width 0.25) (layer "B.Cu") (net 5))
 (segment (start 99.06 64.77) (end 101.346 67.056) (width 0.25) (layer "B.Cu") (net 5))
 (segment (start 101.346 113.735919) (end 99.225479 115.85644) (width 0.25) (layer "B.Cu") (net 5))
 (segment (start 101.346 120.142) (end 101.346 124.714) (width 0.25) (layer "B.Cu") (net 5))
 (segment (start 105.355479 138.375479) (end 105.41 138.43) (width 0.25) (layer "B.Cu") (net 5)))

